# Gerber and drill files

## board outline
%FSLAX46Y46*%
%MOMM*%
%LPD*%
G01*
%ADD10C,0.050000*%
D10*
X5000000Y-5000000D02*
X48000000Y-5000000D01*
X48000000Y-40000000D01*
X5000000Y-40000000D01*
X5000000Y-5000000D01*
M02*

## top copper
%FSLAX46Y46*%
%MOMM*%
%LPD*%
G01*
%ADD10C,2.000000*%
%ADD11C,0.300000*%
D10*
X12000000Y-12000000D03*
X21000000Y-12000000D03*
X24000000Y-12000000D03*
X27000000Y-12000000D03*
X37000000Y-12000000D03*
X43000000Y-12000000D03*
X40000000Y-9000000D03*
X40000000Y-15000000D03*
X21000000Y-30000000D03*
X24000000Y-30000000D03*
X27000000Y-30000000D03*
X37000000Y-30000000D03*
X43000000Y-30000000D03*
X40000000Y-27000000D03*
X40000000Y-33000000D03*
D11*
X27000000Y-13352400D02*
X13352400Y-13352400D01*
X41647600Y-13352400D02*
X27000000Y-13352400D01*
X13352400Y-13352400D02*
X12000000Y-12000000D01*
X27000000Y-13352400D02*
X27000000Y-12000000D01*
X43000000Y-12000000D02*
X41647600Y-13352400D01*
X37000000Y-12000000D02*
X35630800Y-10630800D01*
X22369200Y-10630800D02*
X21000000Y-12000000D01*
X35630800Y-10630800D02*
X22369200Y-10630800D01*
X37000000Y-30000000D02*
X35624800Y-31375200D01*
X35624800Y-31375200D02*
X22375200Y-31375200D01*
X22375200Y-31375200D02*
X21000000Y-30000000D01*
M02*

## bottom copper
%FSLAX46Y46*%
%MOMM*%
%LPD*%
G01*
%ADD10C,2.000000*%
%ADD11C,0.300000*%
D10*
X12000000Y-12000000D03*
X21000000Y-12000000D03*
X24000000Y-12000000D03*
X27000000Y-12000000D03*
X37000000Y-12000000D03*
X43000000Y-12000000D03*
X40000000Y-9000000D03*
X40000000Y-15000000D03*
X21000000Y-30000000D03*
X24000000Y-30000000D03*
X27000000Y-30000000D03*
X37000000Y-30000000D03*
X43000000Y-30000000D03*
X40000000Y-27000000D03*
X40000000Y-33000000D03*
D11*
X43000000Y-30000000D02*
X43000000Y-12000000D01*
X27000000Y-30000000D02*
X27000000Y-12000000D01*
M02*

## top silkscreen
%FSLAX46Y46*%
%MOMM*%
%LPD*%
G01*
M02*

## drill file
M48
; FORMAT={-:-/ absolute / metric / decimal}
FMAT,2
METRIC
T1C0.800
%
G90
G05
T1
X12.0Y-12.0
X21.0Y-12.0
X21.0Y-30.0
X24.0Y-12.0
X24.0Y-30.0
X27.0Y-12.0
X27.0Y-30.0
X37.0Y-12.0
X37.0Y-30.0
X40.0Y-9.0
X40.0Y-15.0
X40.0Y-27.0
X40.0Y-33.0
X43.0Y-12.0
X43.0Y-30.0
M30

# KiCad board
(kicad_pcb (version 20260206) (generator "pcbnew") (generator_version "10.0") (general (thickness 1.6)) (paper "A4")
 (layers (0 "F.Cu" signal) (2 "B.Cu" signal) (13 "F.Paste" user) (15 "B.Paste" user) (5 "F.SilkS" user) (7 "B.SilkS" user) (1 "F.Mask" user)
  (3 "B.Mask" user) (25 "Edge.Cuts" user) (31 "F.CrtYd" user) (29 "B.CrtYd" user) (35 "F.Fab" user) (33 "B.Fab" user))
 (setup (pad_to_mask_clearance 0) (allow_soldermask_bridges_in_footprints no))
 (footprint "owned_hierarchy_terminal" (layer "F.Cu") (at 12 12)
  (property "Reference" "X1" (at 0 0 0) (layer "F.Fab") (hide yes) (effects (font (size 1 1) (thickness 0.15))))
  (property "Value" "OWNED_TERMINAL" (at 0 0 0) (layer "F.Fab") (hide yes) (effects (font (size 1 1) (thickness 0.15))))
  (pad "1" thru_hole circle (at 0 0) (size 2 2) (drill 0.8) (layers "*.Cu" "*.Mask") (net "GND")))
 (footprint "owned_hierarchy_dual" (layer "F.Cu") (at 24 12)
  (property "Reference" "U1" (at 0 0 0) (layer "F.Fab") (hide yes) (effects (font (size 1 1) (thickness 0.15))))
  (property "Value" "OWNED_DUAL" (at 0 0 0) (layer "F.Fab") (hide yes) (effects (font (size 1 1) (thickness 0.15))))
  (pad "1" thru_hole circle (at -3 0) (size 2 2) (drill 0.8) (layers "*.Cu" "*.Mask") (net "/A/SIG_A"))
  (pad "2" thru_hole circle (at 0 0) (size 2 2) (drill 0.8) (layers "*.Cu" "*.Mask") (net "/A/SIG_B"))
  (pad "3" thru_hole circle (at 3 0) (size 2 2) (drill 0.8) (layers "*.Cu" "*.Mask") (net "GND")))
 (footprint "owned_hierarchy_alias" (layer "F.Cu") (at 40 12)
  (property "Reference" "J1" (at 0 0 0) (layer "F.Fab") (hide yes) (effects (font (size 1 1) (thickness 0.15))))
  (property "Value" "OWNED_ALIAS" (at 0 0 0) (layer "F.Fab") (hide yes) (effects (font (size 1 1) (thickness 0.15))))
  (pad "R" thru_hole circle (at -3 0) (size 2 2) (drill 0.8) (layers "*.Cu" "*.Mask") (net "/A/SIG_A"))
  (pad "T" thru_hole circle (at 3 0) (size 2 2) (drill 0.8) (layers "*.Cu" "*.Mask") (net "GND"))
  (pad "MP" thru_hole circle (at 0 -3) (size 2 2) (drill 0.8) (layers "*.Cu" "*.Mask"))
  (pad "MP" thru_hole circle (at 0 3) (size 2 2) (drill 0.8) (layers "*.Cu" "*.Mask")))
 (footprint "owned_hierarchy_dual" (layer "F.Cu") (at 24 30)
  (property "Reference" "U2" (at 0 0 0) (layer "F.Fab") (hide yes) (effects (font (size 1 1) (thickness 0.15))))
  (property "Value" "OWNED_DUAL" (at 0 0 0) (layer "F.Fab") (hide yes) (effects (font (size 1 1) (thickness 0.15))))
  (pad "1" thru_hole circle (at -3 0) (size 2 2) (drill 0.8) (layers "*.Cu" "*.Mask") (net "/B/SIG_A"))
  (pad "2" thru_hole circle (at 0 0) (size 2 2) (drill 0.8) (layers "*.Cu" "*.Mask") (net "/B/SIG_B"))
  (pad "3" thru_hole circle (at 3 0) (size 2 2) (drill 0.8) (layers "*.Cu" "*.Mask") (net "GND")))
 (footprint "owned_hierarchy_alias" (layer "F.Cu") (at 40 30)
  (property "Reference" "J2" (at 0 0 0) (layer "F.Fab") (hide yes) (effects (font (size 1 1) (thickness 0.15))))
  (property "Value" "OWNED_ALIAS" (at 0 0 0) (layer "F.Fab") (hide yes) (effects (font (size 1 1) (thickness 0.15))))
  (pad "R" thru_hole circle (at -3 0) (size 2 2) (drill 0.8) (layers "*.Cu" "*.Mask") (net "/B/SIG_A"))
  (pad "T" thru_hole circle (at 3 0) (size 2 2) (drill 0.8) (layers "*.Cu" "*.Mask") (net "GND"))
  (pad "MP" thru_hole circle (at 0 -3) (size 2 2) (drill 0.8) (layers "*.Cu" "*.Mask"))
  (pad "MP" thru_hole circle (at 0 3) (size 2 2) (drill 0.8) (layers "*.Cu" "*.Mask")))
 (gr_rect (start 5 5) (end 48 40) (stroke (width 0.05) (type default)) (fill none) (layer "Edge.Cuts"))
 (segment (start 27 13.3524) (end 13.3524 13.3524) (width 0.3) (layer "F.Cu") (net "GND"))
 (segment (start 41.6476 13.3524) (end 27 13.3524) (width 0.3) (layer "F.Cu") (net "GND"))
 (segment (start 13.3524 13.3524) (end 12 12) (width 0.3) (layer "F.Cu") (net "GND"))
 (segment (start 27 13.3524) (end 27 12) (width 0.3) (layer "F.Cu") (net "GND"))
 (segment (start 43 12) (end 41.6476 13.3524) (width 0.3) (layer "F.Cu") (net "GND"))
 (segment (start 43 30) (end 43 12) (width 0.3) (layer "B.Cu") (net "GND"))
 (segment (start 27 30) (end 27 12) (width 0.3) (layer "B.Cu") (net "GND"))
 (segment (start 37 12) (end 35.6308 10.6308) (width 0.3) (layer "F.Cu") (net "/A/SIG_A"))
 (segment (start 22.3692 10.6308) (end 21 12) (width 0.3) (layer "F.Cu") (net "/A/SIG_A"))
 (segment (start 35.6308 10.6308) (end 22.3692 10.6308) (width 0.3) (layer "F.Cu") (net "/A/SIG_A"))
 (segment (start 37 30) (end 35.6248 31.3752) (width 0.3) (layer "F.Cu") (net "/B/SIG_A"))
 (segment (start 35.6248 31.3752) (end 22.3752 31.3752) (width 0.3) (layer "F.Cu") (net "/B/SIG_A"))
 (segment (start 22.3752 31.3752) (end 21 30) (width 0.3) (layer "F.Cu") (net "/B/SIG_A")))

